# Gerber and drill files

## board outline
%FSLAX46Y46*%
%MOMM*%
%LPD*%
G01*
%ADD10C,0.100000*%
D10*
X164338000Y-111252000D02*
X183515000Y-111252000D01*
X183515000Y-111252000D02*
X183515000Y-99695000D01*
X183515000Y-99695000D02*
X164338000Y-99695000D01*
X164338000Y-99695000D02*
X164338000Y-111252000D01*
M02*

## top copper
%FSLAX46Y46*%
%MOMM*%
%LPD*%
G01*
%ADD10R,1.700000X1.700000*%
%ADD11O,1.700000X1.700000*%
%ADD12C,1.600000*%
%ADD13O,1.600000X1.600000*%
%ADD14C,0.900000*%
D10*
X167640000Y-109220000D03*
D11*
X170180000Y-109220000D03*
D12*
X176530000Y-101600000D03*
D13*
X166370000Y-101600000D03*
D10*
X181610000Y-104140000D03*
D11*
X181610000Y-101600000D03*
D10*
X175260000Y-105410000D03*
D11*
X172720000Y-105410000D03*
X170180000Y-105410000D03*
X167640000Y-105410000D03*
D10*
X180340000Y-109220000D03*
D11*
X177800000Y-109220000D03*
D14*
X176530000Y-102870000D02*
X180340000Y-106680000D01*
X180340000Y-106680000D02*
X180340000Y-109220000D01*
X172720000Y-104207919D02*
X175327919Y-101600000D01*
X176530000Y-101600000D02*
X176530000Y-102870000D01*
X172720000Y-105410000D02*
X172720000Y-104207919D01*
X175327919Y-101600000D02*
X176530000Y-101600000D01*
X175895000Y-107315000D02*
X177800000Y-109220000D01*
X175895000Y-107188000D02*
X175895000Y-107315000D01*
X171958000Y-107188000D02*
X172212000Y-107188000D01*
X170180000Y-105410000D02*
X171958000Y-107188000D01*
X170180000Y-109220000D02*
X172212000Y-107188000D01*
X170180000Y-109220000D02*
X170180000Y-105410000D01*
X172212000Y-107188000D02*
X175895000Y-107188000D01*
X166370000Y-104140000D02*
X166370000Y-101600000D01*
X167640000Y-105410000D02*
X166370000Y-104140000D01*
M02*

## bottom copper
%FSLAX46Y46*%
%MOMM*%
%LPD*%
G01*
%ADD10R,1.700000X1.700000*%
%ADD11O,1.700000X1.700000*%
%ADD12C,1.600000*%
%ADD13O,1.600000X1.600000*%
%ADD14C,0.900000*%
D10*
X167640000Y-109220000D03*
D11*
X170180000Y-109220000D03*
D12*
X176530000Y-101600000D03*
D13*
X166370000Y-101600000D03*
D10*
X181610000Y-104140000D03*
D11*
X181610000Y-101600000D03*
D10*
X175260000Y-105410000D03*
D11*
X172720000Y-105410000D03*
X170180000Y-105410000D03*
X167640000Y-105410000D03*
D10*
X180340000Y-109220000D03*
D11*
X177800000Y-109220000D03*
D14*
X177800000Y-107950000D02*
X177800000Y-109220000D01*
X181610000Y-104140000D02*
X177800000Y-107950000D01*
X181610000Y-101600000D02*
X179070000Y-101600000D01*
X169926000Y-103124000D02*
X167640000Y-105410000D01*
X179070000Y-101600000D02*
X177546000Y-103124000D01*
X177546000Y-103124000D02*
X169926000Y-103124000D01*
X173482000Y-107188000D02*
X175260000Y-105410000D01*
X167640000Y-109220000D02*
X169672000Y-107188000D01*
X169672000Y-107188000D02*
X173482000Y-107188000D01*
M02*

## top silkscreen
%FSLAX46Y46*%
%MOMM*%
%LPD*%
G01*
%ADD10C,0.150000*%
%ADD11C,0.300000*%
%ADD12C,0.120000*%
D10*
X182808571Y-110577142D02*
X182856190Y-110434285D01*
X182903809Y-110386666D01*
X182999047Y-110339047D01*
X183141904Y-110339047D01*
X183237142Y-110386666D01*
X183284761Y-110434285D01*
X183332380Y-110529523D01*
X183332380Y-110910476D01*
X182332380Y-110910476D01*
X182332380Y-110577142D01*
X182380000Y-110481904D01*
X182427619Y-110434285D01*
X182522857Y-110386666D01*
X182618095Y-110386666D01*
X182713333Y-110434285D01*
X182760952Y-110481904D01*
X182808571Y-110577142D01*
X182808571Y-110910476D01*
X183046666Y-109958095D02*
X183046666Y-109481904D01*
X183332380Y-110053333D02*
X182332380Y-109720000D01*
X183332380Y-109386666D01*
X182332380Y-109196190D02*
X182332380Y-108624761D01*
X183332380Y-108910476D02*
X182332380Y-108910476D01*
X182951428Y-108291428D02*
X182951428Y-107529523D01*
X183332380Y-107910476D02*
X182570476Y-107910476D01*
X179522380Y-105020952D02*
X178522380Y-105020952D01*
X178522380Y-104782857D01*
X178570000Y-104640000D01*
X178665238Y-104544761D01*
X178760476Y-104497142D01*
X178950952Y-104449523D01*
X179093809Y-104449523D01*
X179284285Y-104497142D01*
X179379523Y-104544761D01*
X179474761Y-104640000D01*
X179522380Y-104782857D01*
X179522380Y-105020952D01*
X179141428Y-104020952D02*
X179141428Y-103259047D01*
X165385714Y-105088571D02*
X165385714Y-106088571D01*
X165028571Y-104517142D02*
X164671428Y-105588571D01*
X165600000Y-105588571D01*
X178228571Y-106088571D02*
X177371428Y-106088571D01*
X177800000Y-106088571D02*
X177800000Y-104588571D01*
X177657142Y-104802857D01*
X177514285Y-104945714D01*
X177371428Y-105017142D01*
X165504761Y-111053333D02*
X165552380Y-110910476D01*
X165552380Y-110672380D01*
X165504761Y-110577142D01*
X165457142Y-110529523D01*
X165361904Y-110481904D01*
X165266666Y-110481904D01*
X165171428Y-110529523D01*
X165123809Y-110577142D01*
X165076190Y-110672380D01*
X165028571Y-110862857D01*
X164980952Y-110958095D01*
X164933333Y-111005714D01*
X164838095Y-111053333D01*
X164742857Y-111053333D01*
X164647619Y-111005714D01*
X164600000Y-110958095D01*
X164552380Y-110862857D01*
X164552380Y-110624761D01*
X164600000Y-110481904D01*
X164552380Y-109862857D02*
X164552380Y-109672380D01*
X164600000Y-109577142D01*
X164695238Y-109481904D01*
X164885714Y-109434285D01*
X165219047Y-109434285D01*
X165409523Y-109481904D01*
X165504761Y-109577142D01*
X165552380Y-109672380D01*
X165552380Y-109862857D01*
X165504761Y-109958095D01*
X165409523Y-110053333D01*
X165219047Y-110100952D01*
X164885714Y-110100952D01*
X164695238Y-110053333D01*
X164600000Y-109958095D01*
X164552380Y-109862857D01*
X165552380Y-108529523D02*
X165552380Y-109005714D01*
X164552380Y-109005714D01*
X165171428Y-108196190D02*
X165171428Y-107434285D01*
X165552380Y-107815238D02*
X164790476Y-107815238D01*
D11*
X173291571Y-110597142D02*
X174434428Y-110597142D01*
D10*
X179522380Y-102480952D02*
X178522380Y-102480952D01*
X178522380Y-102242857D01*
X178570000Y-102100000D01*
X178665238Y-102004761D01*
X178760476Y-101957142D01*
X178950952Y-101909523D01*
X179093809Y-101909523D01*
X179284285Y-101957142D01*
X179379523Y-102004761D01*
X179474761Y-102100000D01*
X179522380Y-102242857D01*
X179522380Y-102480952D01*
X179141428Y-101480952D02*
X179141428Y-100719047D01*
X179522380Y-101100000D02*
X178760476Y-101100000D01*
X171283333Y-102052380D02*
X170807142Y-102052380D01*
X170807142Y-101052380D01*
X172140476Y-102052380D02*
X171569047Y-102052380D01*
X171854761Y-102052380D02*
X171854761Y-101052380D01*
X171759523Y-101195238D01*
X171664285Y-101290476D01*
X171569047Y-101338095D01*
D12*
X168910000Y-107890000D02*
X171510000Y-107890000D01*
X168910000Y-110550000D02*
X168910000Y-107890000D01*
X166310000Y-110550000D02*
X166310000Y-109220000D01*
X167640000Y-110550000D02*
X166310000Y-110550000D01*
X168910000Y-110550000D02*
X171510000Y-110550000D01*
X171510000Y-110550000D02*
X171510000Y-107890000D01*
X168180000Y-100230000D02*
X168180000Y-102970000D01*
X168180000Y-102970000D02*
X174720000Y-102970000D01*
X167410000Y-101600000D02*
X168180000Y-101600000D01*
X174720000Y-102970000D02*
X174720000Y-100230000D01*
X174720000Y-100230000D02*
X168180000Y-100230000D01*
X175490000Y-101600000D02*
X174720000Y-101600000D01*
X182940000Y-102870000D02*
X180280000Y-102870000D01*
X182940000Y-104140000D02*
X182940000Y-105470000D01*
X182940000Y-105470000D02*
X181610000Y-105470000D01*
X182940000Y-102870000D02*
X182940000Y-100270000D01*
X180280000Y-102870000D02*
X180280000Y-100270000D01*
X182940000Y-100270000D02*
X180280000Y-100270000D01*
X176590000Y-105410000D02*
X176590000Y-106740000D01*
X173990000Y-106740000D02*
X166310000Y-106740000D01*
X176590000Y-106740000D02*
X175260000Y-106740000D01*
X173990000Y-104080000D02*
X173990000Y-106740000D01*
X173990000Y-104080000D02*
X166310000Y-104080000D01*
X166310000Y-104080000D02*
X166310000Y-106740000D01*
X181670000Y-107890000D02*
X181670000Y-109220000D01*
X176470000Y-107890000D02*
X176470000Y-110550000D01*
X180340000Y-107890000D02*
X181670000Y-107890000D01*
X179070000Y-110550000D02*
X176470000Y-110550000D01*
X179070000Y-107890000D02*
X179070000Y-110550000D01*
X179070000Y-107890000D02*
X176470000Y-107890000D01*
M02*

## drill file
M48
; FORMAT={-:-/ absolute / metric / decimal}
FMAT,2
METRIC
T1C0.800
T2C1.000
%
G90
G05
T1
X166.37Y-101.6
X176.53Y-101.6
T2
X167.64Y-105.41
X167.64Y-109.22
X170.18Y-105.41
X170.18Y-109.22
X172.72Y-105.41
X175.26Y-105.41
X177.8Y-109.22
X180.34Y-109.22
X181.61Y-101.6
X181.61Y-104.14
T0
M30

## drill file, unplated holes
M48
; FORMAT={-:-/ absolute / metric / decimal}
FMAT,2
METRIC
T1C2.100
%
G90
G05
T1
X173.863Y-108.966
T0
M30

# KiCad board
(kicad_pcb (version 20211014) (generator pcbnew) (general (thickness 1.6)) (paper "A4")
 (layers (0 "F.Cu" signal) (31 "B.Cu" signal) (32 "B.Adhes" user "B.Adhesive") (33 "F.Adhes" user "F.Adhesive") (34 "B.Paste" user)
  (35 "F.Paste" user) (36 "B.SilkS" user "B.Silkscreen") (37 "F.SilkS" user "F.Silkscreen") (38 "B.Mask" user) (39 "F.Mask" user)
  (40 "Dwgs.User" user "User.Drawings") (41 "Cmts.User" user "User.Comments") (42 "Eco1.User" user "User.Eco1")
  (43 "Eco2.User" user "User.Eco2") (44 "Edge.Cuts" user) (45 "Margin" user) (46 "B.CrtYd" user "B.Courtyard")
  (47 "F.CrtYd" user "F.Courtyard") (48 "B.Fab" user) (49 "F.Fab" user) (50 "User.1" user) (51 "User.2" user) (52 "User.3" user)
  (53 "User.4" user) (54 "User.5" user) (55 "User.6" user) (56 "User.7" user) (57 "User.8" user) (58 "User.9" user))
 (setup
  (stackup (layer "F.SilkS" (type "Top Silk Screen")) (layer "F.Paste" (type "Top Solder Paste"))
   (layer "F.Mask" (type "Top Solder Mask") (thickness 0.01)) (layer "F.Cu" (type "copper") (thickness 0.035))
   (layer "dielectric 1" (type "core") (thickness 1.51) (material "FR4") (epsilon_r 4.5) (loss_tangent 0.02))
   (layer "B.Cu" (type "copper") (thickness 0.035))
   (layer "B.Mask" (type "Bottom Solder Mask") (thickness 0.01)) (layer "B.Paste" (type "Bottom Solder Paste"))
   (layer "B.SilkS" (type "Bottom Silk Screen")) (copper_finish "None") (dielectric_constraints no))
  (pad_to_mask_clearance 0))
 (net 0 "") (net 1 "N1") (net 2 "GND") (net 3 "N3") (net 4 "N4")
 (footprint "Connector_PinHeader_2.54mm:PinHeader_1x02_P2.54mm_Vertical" (layer "F.Cu") (at 167.64 109.22 90)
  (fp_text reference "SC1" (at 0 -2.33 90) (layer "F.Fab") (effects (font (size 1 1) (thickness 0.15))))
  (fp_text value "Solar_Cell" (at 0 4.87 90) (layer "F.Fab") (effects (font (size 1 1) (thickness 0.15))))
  (fp_line (start 1.33 1.27) (end 1.33 3.87) (layer "F.SilkS") (width 0.12))
  (fp_line (start -1.33 1.27) (end 1.33 1.27) (layer "F.SilkS") (width 0.12))
  (fp_line (start -1.33 -1.33) (end 0 -1.33) (layer "F.SilkS") (width 0.12))
  (fp_line (start -1.33 0) (end -1.33 -1.33) (layer "F.SilkS") (width 0.12))
  (fp_line (start -1.33 1.27) (end -1.33 3.87) (layer "F.SilkS") (width 0.12))
  (fp_line (start -1.33 3.87) (end 1.33 3.87) (layer "F.SilkS") (width 0.12))
  (pad "1" thru_hole rect (at 0 0 90) (size 1.7 1.7) (drill 1) (layers *.Cu *.Mask) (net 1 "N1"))
  (pad "2" thru_hole oval (at 0 2.54 90) (size 1.7 1.7) (drill 1) (layers *.Cu *.Mask) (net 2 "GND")))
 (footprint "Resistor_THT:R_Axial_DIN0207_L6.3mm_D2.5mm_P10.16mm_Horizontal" (layer "F.Cu") (at 176.53 101.6 180)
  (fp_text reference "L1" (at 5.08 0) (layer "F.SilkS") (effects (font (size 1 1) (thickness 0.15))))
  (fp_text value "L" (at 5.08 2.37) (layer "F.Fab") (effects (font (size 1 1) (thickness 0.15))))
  (fp_line (start 8.35 1.37) (end 8.35 -1.37) (layer "F.SilkS") (width 0.12))
  (fp_line (start 8.35 -1.37) (end 1.81 -1.37) (layer "F.SilkS") (width 0.12))
  (fp_line (start 9.12 0) (end 8.35 0) (layer "F.SilkS") (width 0.12))
  (fp_line (start 1.81 -1.37) (end 1.81 1.37) (layer "F.SilkS") (width 0.12))
  (fp_line (start 1.81 1.37) (end 8.35 1.37) (layer "F.SilkS") (width 0.12))
  (fp_line (start 1.04 0) (end 1.81 0) (layer "F.SilkS") (width 0.12))
  (pad "1" thru_hole circle (at 0 0 180) (size 1.6 1.6) (drill 0.8) (layers *.Cu *.Mask) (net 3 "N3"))
  (pad "2" thru_hole oval (at 10.16 0 180) (size 1.6 1.6) (drill 0.8) (layers *.Cu *.Mask) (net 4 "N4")))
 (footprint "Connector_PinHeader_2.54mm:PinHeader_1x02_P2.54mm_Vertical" (layer "F.Cu") (at 181.61 104.14 180)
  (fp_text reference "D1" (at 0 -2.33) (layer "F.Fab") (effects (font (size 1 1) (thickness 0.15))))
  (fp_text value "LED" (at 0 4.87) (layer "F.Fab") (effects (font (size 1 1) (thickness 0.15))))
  (fp_line (start -1.33 1.27) (end 1.33 1.27) (layer "F.SilkS") (width 0.12))
  (fp_line (start -1.33 0) (end -1.33 -1.33) (layer "F.SilkS") (width 0.12))
  (fp_line (start -1.33 -1.33) (end 0 -1.33) (layer "F.SilkS") (width 0.12))
  (fp_line (start -1.33 1.27) (end -1.33 3.87) (layer "F.SilkS") (width 0.12))
  (fp_line (start 1.33 1.27) (end 1.33 3.87) (layer "F.SilkS") (width 0.12))
  (fp_line (start -1.33 3.87) (end 1.33 3.87) (layer "F.SilkS") (width 0.12))
  (pad "1" thru_hole rect (at 0 0 180) (size 1.7 1.7) (drill 1) (layers *.Cu *.Mask) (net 2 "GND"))
  (pad "2" thru_hole oval (at 0 2.54 180) (size 1.7 1.7) (drill 1) (layers *.Cu *.Mask) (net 4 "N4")))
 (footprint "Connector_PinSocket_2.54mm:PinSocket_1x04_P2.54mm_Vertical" (layer "F.Cu") (at 175.26 105.41 -90)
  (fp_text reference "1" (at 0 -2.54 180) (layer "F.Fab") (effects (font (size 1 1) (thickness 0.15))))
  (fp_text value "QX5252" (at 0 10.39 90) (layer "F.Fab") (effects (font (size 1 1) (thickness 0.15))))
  (fp_line (start 0 -1.33) (end 1.33 -1.33) (layer "F.SilkS") (width 0.12))
  (fp_line (start 1.33 1.27) (end 1.33 8.95) (layer "F.SilkS") (width 0.12))
  (fp_line (start 1.33 -1.33) (end 1.33 0) (layer "F.SilkS") (width 0.12))
  (fp_line (start -1.33 1.27) (end 1.33 1.27) (layer "F.SilkS") (width 0.12))
  (fp_line (start -1.33 1.27) (end -1.33 8.95) (layer "F.SilkS") (width 0.12))
  (fp_line (start -1.33 8.95) (end 1.33 8.95) (layer "F.SilkS") (width 0.12))
  (pad "1" thru_hole rect (at 0 0 270) (size 1.7 1.7) (drill 1) (layers *.Cu *.Mask) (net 1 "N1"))
  (pad "2" thru_hole oval (at 0 2.54 270) (size 1.7 1.7) (drill 1) (layers *.Cu *.Mask) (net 3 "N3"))
  (pad "3" thru_hole oval (at 0 5.08 270) (size 1.7 1.7) (drill 1) (layers *.Cu *.Mask) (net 2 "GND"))
  (pad "4" thru_hole oval (at 0 7.62 270) (size 1.7 1.7) (drill 1) (layers *.Cu *.Mask) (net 4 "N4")))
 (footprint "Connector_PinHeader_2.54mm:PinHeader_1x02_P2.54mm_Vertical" (layer "F.Cu") (at 180.34 109.22 -90)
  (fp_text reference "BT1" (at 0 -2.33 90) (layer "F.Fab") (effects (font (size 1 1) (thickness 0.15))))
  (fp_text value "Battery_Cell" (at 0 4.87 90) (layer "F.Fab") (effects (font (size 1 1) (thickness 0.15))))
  (fp_line (start -1.33 -1.33) (end 0 -1.33) (layer "F.SilkS") (width 0.12))
  (fp_line (start -1.33 3.87) (end 1.33 3.87) (layer "F.SilkS") (width 0.12))
  (fp_line (start -1.33 0) (end -1.33 -1.33) (layer "F.SilkS") (width 0.12))
  (fp_line (start 1.33 1.27) (end 1.33 3.87) (layer "F.SilkS") (width 0.12))
  (fp_line (start -1.33 1.27) (end 1.33 1.27) (layer "F.SilkS") (width 0.12))
  (fp_line (start -1.33 1.27) (end -1.33 3.87) (layer "F.SilkS") (width 0.12))
  (pad "1" thru_hole rect (at 0 0 270) (size 1.7 1.7) (drill 1) (layers *.Cu *.Mask) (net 3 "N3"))
  (pad "2" thru_hole oval (at 0 2.54 270) (size 1.7 1.7) (drill 1) (layers *.Cu *.Mask) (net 2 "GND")))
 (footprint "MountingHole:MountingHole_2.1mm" (layer "F.Cu") (at 173.863 108.966)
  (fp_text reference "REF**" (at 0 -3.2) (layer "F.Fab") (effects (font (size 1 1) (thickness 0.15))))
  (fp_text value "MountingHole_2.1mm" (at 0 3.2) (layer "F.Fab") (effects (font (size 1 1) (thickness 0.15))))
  (pad "" np_thru_hole circle (at 0 0) (size 2.1 2.1) (drill 2.1) (layers *.Cu *.Mask)))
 (gr_rect (start 164.338 111.252) (end 183.515 99.695) (layer "Edge.Cuts") (width 0.1) (fill none))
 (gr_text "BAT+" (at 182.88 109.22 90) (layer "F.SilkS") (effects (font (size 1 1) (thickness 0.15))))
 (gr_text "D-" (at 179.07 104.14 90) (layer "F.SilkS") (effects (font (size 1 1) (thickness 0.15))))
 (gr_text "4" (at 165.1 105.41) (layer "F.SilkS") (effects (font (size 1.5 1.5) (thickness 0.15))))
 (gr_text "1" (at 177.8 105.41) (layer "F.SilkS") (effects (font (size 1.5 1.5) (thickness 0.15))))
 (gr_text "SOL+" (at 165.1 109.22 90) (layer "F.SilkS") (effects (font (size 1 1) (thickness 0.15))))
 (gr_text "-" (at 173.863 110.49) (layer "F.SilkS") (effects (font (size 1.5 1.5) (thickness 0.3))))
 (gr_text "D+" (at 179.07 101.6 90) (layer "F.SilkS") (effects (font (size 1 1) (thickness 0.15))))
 (segment (start 176.53 102.87) (end 180.34 106.68) (width 0.9) (layer "F.Cu") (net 3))
 (segment (start 180.34 106.68) (end 180.34 109.22) (width 0.9) (layer "F.Cu") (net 3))
 (segment (start 172.72 104.207919) (end 175.327919 101.6) (width 0.9) (layer "F.Cu") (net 3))
 (segment (start 176.53 101.6) (end 176.53 102.87) (width 0.9) (layer "F.Cu") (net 3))
 (segment (start 172.72 105.41) (end 172.72 104.207919) (width 0.9) (layer "F.Cu") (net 3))
 (segment (start 175.327919 101.6) (end 176.53 101.6) (width 0.9) (layer "F.Cu") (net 3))
 (segment (start 175.895 107.315) (end 177.8 109.22) (width 0.9) (layer "F.Cu") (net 2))
 (segment (start 175.895 107.188) (end 175.895 107.315) (width 0.9) (layer "F.Cu") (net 2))
 (segment (start 171.958 107.188) (end 172.212 107.188) (width 0.9) (layer "F.Cu") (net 2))
 (segment (start 170.18 105.41) (end 171.958 107.188) (width 0.9) (layer "F.Cu") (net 2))
 (segment (start 170.18 109.22) (end 172.212 107.188) (width 0.9) (layer "F.Cu") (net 2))
 (segment (start 170.18 109.22) (end 170.18 105.41) (width 0.9) (layer "F.Cu") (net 2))
 (segment (start 172.212 107.188) (end 175.895 107.188) (width 0.9) (layer "F.Cu") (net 2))
 (segment (start 177.8 107.95) (end 177.8 109.22) (width 0.9) (layer "B.Cu") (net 2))
 (segment (start 181.61 104.14) (end 177.8 107.95) (width 0.9) (layer "B.Cu") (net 2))
 (segment (start 166.37 104.14) (end 166.37 101.6) (width 0.9) (layer "F.Cu") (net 4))
 (segment (start 167.64 105.41) (end 166.37 104.14) (width 0.9) (layer "F.Cu") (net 4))
 (segment (start 181.61 101.6) (end 179.07 101.6) (width 0.9) (layer "B.Cu") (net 4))
 (segment (start 169.926 103.124) (end 167.64 105.41) (width 0.9) (layer "B.Cu") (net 4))
 (segment (start 179.07 101.6) (end 177.546 103.124) (width 0.9) (layer "B.Cu") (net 4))
 (segment (start 177.546 103.124) (end 169.926 103.124) (width 0.9) (layer "B.Cu") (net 4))
 (segment (start 173.482 107.188) (end 175.26 105.41) (width 0.9) (layer "B.Cu") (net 1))
 (segment (start 167.64 109.22) (end 169.672 107.188) (width 0.9) (layer "B.Cu") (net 1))
 (segment (start 169.672 107.188) (end 173.482 107.188) (width 0.9) (layer "B.Cu") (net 1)))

